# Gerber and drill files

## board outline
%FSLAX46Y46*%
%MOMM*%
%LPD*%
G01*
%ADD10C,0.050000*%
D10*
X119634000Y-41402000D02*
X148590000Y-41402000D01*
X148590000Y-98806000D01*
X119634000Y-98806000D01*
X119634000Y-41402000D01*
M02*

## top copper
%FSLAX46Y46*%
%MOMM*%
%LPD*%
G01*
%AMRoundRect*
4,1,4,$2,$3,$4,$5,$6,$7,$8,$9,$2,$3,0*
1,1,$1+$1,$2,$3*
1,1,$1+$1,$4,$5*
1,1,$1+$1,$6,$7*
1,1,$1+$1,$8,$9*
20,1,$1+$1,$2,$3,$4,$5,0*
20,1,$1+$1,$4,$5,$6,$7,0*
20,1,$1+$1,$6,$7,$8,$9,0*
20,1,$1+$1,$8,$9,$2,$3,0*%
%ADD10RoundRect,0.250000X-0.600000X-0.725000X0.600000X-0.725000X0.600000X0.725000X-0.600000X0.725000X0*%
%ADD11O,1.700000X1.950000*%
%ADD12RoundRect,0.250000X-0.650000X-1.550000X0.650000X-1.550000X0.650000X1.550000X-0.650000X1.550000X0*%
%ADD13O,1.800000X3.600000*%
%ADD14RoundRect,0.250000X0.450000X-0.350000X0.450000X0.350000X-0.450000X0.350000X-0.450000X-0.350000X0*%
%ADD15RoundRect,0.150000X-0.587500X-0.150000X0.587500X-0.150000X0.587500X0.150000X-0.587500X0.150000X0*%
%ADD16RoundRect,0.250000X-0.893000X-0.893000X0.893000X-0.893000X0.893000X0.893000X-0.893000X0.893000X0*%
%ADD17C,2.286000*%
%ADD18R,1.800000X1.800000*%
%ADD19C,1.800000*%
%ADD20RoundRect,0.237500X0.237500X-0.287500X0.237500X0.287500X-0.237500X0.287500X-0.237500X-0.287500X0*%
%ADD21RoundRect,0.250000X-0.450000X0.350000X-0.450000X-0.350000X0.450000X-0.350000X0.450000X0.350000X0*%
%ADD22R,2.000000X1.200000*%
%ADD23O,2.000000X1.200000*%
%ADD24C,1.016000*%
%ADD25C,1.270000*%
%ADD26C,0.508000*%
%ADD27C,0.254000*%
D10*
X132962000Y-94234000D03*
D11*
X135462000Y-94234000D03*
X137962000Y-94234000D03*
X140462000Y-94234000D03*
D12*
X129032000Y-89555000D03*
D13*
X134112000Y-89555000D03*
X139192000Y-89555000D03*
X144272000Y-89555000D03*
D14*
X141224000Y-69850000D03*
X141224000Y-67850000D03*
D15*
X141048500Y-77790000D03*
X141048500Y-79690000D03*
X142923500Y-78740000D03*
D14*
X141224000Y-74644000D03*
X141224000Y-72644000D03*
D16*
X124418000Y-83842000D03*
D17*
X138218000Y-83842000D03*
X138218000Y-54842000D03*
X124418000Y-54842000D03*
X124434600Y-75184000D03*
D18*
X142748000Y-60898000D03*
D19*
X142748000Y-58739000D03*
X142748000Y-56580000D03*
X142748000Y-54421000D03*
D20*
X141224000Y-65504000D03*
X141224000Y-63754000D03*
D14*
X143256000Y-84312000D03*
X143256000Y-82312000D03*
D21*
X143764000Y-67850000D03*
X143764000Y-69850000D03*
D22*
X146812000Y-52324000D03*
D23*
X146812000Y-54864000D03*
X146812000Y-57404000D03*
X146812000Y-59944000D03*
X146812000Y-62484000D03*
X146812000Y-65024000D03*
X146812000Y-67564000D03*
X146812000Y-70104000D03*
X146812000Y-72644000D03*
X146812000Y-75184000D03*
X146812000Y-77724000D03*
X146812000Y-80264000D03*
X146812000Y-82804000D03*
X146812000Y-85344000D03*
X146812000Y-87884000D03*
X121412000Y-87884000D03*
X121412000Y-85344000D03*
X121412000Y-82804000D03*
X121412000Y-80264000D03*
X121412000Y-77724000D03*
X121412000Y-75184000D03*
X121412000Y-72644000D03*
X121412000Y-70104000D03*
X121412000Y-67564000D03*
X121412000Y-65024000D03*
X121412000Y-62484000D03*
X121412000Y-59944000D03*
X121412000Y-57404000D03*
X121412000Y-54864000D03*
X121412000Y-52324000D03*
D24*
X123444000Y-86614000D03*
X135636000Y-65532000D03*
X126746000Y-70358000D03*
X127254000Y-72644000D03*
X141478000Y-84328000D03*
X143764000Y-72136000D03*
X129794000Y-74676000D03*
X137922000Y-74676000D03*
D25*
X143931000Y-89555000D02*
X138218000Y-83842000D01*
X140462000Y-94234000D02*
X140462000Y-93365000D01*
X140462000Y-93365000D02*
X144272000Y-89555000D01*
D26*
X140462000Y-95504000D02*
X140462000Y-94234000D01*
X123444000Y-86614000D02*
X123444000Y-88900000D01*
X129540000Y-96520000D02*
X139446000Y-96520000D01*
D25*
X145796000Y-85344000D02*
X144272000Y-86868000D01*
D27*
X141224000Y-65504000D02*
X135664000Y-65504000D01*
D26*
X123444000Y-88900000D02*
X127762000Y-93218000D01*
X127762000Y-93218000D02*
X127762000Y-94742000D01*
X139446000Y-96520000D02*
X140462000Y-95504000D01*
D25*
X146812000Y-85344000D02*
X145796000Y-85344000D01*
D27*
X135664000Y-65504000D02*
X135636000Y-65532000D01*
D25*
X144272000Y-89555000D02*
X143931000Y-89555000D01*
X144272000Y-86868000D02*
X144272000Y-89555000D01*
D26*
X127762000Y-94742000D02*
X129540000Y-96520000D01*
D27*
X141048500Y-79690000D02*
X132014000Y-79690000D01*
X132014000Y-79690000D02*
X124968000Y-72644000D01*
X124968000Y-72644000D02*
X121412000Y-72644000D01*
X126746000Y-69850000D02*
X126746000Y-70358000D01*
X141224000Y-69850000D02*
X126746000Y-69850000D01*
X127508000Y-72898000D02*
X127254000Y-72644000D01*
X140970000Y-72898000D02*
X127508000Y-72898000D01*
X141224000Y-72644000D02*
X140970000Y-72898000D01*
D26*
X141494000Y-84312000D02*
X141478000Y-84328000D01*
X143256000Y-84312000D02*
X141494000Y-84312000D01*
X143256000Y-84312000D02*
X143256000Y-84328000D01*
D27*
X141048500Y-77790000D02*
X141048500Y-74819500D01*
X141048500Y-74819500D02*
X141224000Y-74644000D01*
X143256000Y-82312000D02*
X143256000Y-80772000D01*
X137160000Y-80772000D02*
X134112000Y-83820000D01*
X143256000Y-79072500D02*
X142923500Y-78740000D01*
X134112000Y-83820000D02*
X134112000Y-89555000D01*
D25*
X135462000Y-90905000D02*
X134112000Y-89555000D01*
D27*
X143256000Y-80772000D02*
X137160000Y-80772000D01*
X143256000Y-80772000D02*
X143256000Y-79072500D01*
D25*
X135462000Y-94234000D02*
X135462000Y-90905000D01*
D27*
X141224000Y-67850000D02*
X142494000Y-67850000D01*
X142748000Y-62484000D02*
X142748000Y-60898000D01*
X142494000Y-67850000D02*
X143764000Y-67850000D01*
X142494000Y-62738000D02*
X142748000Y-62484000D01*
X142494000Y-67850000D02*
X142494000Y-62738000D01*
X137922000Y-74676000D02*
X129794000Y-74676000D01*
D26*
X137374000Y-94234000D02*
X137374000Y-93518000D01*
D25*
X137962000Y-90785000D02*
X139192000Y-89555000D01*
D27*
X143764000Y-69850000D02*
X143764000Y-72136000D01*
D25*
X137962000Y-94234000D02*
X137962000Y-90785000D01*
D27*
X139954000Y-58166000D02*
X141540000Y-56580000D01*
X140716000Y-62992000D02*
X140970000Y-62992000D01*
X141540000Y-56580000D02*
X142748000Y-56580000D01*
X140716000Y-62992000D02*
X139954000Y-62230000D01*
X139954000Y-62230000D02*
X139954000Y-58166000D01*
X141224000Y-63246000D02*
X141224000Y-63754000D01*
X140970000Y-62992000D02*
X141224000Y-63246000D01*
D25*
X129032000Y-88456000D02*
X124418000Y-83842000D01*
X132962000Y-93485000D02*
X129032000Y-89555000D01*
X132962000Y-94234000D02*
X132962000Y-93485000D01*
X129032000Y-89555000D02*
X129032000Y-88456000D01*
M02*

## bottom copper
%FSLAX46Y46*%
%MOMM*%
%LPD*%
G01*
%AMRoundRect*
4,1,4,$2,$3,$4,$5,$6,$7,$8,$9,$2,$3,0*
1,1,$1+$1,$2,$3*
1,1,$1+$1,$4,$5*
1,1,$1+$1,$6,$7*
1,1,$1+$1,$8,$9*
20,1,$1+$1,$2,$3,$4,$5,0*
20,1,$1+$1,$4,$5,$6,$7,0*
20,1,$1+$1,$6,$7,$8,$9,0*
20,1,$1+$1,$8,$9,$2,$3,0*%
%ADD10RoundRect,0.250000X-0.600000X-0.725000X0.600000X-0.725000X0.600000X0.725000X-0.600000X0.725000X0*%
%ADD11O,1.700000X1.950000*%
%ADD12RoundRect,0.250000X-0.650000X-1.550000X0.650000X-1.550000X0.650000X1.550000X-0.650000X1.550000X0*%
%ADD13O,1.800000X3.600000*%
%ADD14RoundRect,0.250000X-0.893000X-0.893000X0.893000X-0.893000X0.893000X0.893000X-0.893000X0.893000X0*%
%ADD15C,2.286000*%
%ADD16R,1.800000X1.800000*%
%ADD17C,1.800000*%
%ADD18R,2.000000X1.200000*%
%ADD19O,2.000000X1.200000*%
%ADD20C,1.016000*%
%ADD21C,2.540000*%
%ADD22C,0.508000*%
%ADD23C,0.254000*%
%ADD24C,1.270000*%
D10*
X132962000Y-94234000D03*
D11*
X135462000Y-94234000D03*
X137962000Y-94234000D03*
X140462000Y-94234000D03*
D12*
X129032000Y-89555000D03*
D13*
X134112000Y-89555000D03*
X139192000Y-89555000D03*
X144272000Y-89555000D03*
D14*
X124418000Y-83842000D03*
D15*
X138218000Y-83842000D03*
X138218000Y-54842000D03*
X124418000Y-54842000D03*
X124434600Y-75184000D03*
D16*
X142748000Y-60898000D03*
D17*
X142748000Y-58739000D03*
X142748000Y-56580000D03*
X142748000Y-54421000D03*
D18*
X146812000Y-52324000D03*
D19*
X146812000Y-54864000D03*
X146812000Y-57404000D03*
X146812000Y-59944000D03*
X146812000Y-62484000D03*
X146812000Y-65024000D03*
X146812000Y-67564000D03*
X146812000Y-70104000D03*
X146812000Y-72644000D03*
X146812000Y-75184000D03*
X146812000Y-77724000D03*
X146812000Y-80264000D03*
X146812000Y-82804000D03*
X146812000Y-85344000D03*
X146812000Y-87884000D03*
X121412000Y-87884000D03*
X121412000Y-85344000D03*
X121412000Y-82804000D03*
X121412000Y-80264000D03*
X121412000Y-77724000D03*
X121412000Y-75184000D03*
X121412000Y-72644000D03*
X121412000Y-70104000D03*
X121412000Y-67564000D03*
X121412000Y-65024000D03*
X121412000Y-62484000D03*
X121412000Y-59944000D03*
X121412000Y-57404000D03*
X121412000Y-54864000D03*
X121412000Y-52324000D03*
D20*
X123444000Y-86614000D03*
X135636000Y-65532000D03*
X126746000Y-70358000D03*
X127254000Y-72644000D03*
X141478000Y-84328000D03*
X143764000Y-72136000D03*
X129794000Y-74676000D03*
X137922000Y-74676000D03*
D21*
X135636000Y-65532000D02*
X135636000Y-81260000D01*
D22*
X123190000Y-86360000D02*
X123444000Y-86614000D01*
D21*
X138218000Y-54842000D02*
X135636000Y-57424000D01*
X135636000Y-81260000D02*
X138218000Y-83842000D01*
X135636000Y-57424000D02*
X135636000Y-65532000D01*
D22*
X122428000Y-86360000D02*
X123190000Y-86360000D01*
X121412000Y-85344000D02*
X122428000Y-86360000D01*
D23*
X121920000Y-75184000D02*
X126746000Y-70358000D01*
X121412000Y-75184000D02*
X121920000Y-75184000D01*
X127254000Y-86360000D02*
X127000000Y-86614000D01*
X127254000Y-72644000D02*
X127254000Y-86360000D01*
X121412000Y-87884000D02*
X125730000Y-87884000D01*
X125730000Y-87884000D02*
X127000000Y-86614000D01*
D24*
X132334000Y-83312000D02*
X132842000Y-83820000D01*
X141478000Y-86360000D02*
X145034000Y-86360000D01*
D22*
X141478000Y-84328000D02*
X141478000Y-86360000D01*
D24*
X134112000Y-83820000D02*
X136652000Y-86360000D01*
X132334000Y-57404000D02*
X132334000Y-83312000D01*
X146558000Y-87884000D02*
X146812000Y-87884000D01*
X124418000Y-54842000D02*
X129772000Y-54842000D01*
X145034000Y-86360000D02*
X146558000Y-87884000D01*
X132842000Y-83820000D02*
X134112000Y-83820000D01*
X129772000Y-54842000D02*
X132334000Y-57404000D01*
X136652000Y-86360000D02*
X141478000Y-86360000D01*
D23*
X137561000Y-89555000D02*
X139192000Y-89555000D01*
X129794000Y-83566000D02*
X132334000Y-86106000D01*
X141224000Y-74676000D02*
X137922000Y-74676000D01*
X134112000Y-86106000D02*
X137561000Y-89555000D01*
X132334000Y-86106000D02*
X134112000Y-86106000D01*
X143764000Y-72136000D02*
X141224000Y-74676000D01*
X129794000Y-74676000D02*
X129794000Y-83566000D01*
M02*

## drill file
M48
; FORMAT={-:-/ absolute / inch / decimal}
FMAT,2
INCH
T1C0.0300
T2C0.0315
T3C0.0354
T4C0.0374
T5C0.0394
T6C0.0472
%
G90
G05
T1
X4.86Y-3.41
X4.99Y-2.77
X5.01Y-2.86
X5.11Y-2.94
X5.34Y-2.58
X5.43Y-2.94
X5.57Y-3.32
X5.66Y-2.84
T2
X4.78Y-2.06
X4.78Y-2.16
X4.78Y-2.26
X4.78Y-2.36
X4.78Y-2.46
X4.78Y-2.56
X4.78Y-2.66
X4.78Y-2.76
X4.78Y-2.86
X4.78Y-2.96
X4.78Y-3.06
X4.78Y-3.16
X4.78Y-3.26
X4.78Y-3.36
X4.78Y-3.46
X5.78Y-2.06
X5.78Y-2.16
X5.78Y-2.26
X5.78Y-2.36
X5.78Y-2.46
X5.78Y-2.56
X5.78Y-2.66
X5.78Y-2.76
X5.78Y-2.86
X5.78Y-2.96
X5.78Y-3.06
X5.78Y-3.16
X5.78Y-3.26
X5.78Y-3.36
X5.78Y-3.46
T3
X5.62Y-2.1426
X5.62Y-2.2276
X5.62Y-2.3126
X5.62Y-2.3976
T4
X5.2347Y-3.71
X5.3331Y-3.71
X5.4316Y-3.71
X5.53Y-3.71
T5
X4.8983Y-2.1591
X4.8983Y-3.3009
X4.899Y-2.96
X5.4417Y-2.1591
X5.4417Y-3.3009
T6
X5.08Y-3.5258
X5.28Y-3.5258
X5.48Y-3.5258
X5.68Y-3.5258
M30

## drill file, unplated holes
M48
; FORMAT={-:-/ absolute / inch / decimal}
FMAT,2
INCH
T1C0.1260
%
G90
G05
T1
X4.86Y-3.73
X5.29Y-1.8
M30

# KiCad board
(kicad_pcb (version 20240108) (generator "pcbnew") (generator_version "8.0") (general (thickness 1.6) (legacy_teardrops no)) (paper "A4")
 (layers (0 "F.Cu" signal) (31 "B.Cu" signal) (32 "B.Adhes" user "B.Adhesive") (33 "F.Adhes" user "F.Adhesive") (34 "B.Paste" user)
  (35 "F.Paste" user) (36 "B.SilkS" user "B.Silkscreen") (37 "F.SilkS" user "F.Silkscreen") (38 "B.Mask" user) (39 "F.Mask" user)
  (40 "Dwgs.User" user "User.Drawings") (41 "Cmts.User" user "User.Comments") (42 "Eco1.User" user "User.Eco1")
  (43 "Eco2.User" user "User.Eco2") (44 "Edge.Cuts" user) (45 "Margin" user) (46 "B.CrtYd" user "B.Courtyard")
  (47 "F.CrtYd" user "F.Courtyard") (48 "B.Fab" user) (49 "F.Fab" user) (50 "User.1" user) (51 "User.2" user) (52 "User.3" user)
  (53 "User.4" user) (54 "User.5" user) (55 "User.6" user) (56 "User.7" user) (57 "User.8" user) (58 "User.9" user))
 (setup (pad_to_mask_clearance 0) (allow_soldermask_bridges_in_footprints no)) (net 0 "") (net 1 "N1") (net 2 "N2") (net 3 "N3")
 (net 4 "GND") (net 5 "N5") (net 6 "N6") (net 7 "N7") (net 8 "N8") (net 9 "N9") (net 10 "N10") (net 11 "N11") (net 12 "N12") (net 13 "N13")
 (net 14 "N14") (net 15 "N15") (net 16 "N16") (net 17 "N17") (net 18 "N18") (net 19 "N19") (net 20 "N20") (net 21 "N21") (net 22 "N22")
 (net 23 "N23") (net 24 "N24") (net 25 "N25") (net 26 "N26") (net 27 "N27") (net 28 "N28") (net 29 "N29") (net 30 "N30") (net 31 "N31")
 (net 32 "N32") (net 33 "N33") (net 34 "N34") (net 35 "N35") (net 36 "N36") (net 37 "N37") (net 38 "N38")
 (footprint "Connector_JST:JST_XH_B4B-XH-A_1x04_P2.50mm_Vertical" (layer "F.Cu") (at 132.962 94.234)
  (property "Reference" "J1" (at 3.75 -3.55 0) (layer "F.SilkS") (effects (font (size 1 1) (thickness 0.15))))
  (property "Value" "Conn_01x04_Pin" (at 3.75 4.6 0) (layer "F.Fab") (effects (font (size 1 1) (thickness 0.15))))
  (pad "1" thru_hole roundrect (at 0 0) (size 1.7 1.95) (drill 0.95) (layers "*.Cu" "*.Mask") (remove_unused_layers no)
   (roundrect_rratio 0.147059) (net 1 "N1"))
  (pad "2" thru_hole oval (at 2.5 0) (size 1.7 1.95) (drill 0.95) (layers "*.Cu" "*.Mask") (remove_unused_layers no) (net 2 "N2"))
  (pad "3" thru_hole oval (at 5 0) (size 1.7 1.95) (drill 0.95) (layers "*.Cu" "*.Mask") (remove_unused_layers no) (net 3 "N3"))
  (pad "4" thru_hole oval (at 7.5 0) (size 1.7 1.95) (drill 0.95) (layers "*.Cu" "*.Mask") (remove_unused_layers no) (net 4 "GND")))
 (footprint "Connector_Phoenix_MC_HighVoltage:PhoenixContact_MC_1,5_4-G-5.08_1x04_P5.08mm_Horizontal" (layer "F.Cu") (at 129.032 89.555)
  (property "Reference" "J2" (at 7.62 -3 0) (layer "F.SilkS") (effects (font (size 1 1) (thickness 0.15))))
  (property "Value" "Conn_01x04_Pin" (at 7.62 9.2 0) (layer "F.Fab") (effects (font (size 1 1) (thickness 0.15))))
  (pad "1" thru_hole roundrect (at 0 0) (size 1.8 3.6) (drill 1.2) (layers "*.Cu" "*.Mask") (remove_unused_layers no)
   (roundrect_rratio 0.138889) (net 1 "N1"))
  (pad "2" thru_hole oval (at 5.08 0) (size 1.8 3.6) (drill 1.2) (layers "*.Cu" "*.Mask") (remove_unused_layers no) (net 2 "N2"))
  (pad "3" thru_hole oval (at 10.16 0) (size 1.8 3.6) (drill 1.2) (layers "*.Cu" "*.Mask") (remove_unused_layers no) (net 3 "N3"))
  (pad "4" thru_hole oval (at 15.24 0) (size 1.8 3.6) (drill 1.2) (layers "*.Cu" "*.Mask") (remove_unused_layers no) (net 4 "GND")))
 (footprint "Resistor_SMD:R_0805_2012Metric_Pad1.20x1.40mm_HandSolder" (layer "F.Cu") (at 141.224 68.85 90)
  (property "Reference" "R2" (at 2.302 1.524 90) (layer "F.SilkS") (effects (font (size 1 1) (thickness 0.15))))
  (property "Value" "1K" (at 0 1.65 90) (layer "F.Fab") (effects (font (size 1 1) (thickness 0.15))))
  (pad "1" smd roundrect (at -1 0 90) (size 1.2 1.4) (layers "F.Cu" "F.Paste" "F.Mask") (roundrect_rratio 0.208333) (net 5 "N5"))
  (pad "2" smd roundrect (at 1 0 90) (size 1.2 1.4) (layers "F.Cu" "F.Paste" "F.Mask") (roundrect_rratio 0.208333) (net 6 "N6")))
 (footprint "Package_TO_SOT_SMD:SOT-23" (layer "F.Cu") (at 141.986 78.74)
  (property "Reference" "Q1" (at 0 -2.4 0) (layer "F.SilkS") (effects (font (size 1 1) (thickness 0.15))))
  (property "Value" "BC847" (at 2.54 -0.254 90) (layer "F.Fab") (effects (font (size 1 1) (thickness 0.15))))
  (pad "1" smd roundrect (at -0.9375 -0.95) (size 1.475 0.6) (layers "F.Cu" "F.Paste" "F.Mask") (roundrect_rratio 0.25) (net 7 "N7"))
  (pad "2" smd roundrect (at -0.9375 0.95) (size 1.475 0.6) (layers "F.Cu" "F.Paste" "F.Mask") (roundrect_rratio 0.25) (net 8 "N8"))
  (pad "3" smd roundrect (at 0.9375 0) (size 1.475 0.6) (layers "F.Cu" "F.Paste" "F.Mask") (roundrect_rratio 0.25) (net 2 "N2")))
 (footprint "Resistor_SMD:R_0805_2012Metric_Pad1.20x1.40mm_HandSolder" (layer "F.Cu") (at 141.224 73.644 90)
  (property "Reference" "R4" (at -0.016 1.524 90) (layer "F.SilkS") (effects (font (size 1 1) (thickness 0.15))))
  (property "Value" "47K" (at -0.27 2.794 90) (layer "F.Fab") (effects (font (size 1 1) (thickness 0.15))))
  (pad "1" smd roundrect (at -1 0 90) (size 1.2 1.4) (layers "F.Cu" "F.Paste" "F.Mask") (roundrect_rratio 0.208333) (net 7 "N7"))
  (pad "2" smd roundrect (at 1 0 90) (size 1.2 1.4) (layers "F.Cu" "F.Paste" "F.Mask") (roundrect_rratio 0.208333) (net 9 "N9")))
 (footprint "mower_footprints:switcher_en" (layer "F.Cu") (at 131.318 69.342)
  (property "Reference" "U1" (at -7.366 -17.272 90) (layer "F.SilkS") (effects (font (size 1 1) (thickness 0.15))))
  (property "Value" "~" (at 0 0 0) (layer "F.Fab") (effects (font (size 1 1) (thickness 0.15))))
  (pad "1" thru_hole roundrect (at -6.9 14.5) (size 2.286 2.286) (drill 1) (layers "*.Cu" "*.Mask") (remove_unused_layers no)
   (roundrect_rratio 0.1093613298) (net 1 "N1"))
  (pad "2" thru_hole circle (at 6.9 14.5) (size 2.286 2.286) (drill 1) (layers "*.Cu" "*.Mask") (remove_unused_layers no) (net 4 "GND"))
  (pad "3" thru_hole circle (at 6.9 -14.5) (size 2.286 2.286) (drill 1) (layers "*.Cu" "*.Mask") (remove_unused_layers no) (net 4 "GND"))
  (pad "4" thru_hole circle (at -6.9 -14.5) (size 2.286 2.286) (drill 1) (layers "*.Cu" "*.Mask") (remove_unused_layers no) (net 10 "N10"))
  (pad "5" thru_hole circle (at -6.8834 5.842) (size 2.286 2.286) (drill 1) (layers "*.Cu" "*.Mask") (remove_unused_layers no)
   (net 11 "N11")))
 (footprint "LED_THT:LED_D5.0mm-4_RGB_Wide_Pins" (layer "F.Cu") (at 142.748 60.898 90)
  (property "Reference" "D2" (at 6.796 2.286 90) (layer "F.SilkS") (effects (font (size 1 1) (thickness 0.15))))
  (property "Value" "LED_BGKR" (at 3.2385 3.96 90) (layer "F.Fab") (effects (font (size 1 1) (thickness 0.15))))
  (pad "1" thru_hole rect (at 0 0 90) (size 1.8 1.8) (drill 0.9) (layers "*.Cu" "*.Mask") (remove_unused_layers no) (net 6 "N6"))
  (pad "2" thru_hole circle (at 2.159 0 90) (size 1.8 1.8) (drill 0.9) (layers "*.Cu" "*.Mask") (remove_unused_layers no) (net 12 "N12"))
  (pad "3" thru_hole circle (at 4.318 0 90) (size 1.8 1.8) (drill 0.9) (layers "*.Cu" "*.Mask") (remove_unused_layers no) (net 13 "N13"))
  (pad "4" thru_hole circle (at 6.477 0 90) (size 1.8 1.8) (drill 0.9) (layers "*.Cu" "*.Mask") (remove_unused_layers no) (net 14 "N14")))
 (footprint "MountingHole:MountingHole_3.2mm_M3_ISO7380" (layer "F.Cu") (at 134.366 45.72)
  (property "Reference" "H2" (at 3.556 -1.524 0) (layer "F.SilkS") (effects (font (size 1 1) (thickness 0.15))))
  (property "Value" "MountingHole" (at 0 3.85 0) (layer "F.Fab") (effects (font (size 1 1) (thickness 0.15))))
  (pad "" np_thru_hole circle (at 0 0) (size 3.2 3.2) (drill 3.2) (layers "*.Cu" "*.Mask")))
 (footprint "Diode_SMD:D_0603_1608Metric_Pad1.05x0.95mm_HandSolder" (layer "F.Cu") (at 141.224 64.629 90)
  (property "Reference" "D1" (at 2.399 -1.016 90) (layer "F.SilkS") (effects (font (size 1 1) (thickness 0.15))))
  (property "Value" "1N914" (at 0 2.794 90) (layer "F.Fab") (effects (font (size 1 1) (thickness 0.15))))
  (pad "1" smd roundrect (at -0.875 0 90) (size 1.05 0.95) (layers "F.Cu" "F.Paste" "F.Mask") (roundrect_rratio 0.25) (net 4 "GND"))
  (pad "2" smd roundrect (at 0.875 0 90) (size 1.05 0.95) (layers "F.Cu" "F.Paste" "F.Mask") (roundrect_rratio 0.25) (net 13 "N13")))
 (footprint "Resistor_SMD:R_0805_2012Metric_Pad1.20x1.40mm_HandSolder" (layer "F.Cu") (at 143.256 83.312 90)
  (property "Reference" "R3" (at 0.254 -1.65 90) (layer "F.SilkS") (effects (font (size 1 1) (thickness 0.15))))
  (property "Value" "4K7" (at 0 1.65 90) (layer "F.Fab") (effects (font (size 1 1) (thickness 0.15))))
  (pad "1" smd roundrect (at -1 0 90) (size 1.2 1.4) (layers "F.Cu" "F.Paste" "F.Mask") (roundrect_rratio 0.208333) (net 10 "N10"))
  (pad "2" smd roundrect (at 1 0 90) (size 1.2 1.4) (layers "F.Cu" "F.Paste" "F.Mask") (roundrect_rratio 0.208333) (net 2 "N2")))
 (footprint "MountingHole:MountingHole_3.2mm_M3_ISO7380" (layer "F.Cu") (at 123.444 94.742)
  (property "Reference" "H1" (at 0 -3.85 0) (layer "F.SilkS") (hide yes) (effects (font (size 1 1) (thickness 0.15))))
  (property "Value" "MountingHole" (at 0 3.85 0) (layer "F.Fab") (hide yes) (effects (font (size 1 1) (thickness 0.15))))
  (pad "" np_thru_hole circle (at 0 0) (size 3.2 3.2) (drill 3.2) (layers "*.Cu" "*.Mask")))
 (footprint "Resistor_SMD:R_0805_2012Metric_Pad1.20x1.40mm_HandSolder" (layer "F.Cu") (at 143.764 68.85 -90)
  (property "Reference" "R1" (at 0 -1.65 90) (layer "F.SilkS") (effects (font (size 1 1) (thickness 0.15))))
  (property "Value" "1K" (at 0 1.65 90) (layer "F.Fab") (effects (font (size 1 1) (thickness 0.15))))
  (pad "1" smd roundrect (at -1 0 270) (size 1.2 1.4) (layers "F.Cu" "F.Paste" "F.Mask") (roundrect_rratio 0.208333) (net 6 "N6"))
  (pad "2" smd roundrect (at 1 0 270) (size 1.2 1.4) (layers "F.Cu" "F.Paste" "F.Mask") (roundrect_rratio 0.208333) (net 3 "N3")))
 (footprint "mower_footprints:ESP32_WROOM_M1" (layer "B.Cu") (at 134.112 70.104 -90)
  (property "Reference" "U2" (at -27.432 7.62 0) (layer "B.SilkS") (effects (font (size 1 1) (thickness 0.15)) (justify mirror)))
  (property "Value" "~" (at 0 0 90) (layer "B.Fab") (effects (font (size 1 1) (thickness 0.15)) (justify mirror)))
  (pad "1" thru_hole rect (at -17.78 -12.7 270) (size 1.2 2) (drill 0.8) (layers "*.Cu" "*.Mask") (remove_unused_layers no) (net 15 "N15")
   (thermal_bridge_angle 45))
  (pad "2" thru_hole oval (at -15.24 -12.7 270) (size 1.2 2) (drill 0.8) (layers "*.Cu" "*.Mask") (remove_unused_layers no) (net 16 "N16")
   (thermal_bridge_angle 45))
  (pad "3" thru_hole oval (at -12.7 -12.7 270) (size 1.2 2) (drill 0.8) (layers "*.Cu" "*.Mask") (remove_unused_layers no) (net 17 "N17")
   (thermal_bridge_angle 45))
  (pad "4" thru_hole oval (at -10.16 -12.7 270) (size 1.2 2) (drill 0.8) (layers "*.Cu" "*.Mask") (remove_unused_layers no) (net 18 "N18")
   (thermal_bridge_angle 45))
  (pad "5" thru_hole oval (at -7.62 -12.7 270) (size 1.2 2) (drill 0.8) (layers "*.Cu" "*.Mask") (remove_unused_layers no) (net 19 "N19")
   (thermal_bridge_angle 45))
  (pad "6" thru_hole oval (at -5.08 -12.7 270) (size 1.2 2) (drill 0.8) (layers "*.Cu" "*.Mask") (remove_unused_layers no) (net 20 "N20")
   (thermal_bridge_angle 45))
  (pad "7" thru_hole oval (at -2.54 -12.7 270) (size 1.2 2) (drill 0.8) (layers "*.Cu" "*.Mask") (remove_unused_layers no) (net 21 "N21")
   (thermal_bridge_angle 45))
  (pad "8" thru_hole oval (at 0 -12.7 270) (size 1.2 2) (drill 0.8) (layers "*.Cu" "*.Mask") (remove_unused_layers no) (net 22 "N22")
   (thermal_bridge_angle 45))
  (pad "9" thru_hole oval (at 2.54 -12.7 270) (size 1.2 2) (drill 0.8) (layers "*.Cu" "*.Mask") (remove_unused_layers no) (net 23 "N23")
   (thermal_bridge_angle 45))
  (pad "10" thru_hole oval (at 5.08 -12.7 270) (size 1.2 2) (drill 0.8) (layers "*.Cu" "*.Mask") (remove_unused_layers no) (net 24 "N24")
   (thermal_bridge_angle 45))
  (pad "11" thru_hole oval (at 7.62 -12.7 270) (size 1.2 2) (drill 0.8) (layers "*.Cu" "*.Mask") (remove_unused_layers no) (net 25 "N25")
   (thermal_bridge_angle 45))
  (pad "12" thru_hole oval (at 10.16 -12.7 270) (size 1.2 2) (drill 0.8) (layers "*.Cu" "*.Mask") (remove_unused_layers no) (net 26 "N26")
   (thermal_bridge_angle 45))
  (pad "13" thru_hole oval (at 12.7 -12.7 270) (size 1.2 2) (drill 0.8) (layers "*.Cu" "*.Mask") (remove_unused_layers no) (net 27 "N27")
   (thermal_bridge_angle 45))
  (pad "14" thru_hole oval (at 15.24 -12.7 270) (size 1.2 2) (drill 0.8) (layers "*.Cu" "*.Mask") (remove_unused_layers no) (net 4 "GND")
   (thermal_bridge_angle 45))
  (pad "15" thru_hole oval (at 17.78 -12.7 270) (size 1.2 2) (drill 0.8) (layers "*.Cu" "*.Mask") (remove_unused_layers no) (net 10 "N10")
   (thermal_bridge_angle 45))
  (pad "16" thru_hole oval (at 17.78 12.7 270) (size 1.2 2) (drill 0.8) (layers "*.Cu" "*.Mask") (remove_unused_layers no) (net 9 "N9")
   (thermal_bridge_angle 45))
  (pad "17" thru_hole oval (at 15.24 12.7 270) (size 1.2 2) (drill 0.8) (layers "*.Cu" "*.Mask") (remove_unused_layers no) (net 4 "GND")
   (thermal_bridge_angle 45))
  (pad "18" thru_hole oval (at 12.7 12.7 270) (size 1.2 2) (drill 0.8) (layers "*.Cu" "*.Mask") (remove_unused_layers no) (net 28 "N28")
   (thermal_bridge_angle 45))
  (pad "19" thru_hole oval (at 10.16 12.7 270) (size 1.2 2) (drill 0.8) (layers "*.Cu" "*.Mask") (remove_unused_layers no) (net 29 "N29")
   (thermal_bridge_angle 45))
  (pad "20" thru_hole oval (at 7.62 12.7 270) (size 1.2 2) (drill 0.8) (layers "*.Cu" "*.Mask") (remove_unused_layers no) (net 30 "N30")
   (thermal_bridge_angle 45))
  (pad "21" thru_hole oval (at 5.08 12.7 270) (size 1.2 2) (drill 0.8) (layers "*.Cu" "*.Mask") (remove_unused_layers no) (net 5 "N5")
   (thermal_bridge_angle 45))
  (pad "22" thru_hole oval (at 2.54 12.7 270) (size 1.2 2) (drill 0.8) (layers "*.Cu" "*.Mask") (remove_unused_layers no) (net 8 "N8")
   (thermal_bridge_angle 45))
  (pad "23" thru_hole oval (at 0 12.7 270) (size 1.2 2) (drill 0.8) (layers "*.Cu" "*.Mask") (remove_unused_layers no) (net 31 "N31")
   (thermal_bridge_angle 45))
  (pad "24" thru_hole oval (at -2.54 12.7 270) (size 1.2 2) (drill 0.8) (layers "*.Cu" "*.Mask") (remove_unused_layers no) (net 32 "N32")
   (thermal_bridge_angle 45))
  (pad "25" thru_hole oval (at -5.08 12.7 270) (size 1.2 2) (drill 0.8) (layers "*.Cu" "*.Mask") (remove_unused_layers no) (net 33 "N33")
   (thermal_bridge_angle 45))
  (pad "26" thru_hole oval (at -7.62 12.7 270) (size 1.2 2) (drill 0.8) (layers "*.Cu" "*.Mask") (remove_unused_layers no) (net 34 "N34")
   (thermal_bridge_angle 45))
  (pad "27" thru_hole oval (at -10.16 12.7 270) (size 1.2 2) (drill 0.8) (layers "*.Cu" "*.Mask") (remove_unused_layers no) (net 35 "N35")
   (thermal_bridge_angle 45))
  (pad "28" thru_hole oval (at -12.7 12.7 270) (size 1.2 2) (drill 0.8) (layers "*.Cu" "*.Mask") (remove_unused_layers no) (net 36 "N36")
   (thermal_bridge_angle 45))
  (pad "29" thru_hole oval (at -15.24 12.7 270) (size 1.2 2) (drill 0.8) (layers "*.Cu" "*.Mask") (remove_unused_layers no) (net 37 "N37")
   (thermal_bridge_angle 45))
  (pad "30" thru_hole oval (at -17.78 12.7 270) (size 1.2 2) (drill 0.8) (layers "*.Cu" "*.Mask") (remove_unused_layers no) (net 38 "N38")
   (thermal_bridge_angle 45)))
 (gr_rect (start 119.634 41.402) (end 148.59 98.806) (stroke (width 0.05) (type default)) (fill none) (layer "Edge.Cuts"))
 (segment (start 143.931 89.555) (end 138.218 83.842) (width 1.27) (layer "F.Cu") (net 4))
 (segment (start 140.462 94.234) (end 140.462 93.365) (width 1.27) (layer "F.Cu") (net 4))
 (segment (start 140.462 93.365) (end 144.272 89.555) (width 1.27) (layer "F.Cu") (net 4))
 (segment (start 140.462 95.504) (end 140.462 94.234) (width 0.508) (layer "F.Cu") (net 4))
 (segment (start 123.444 86.614) (end 123.444 88.9) (width 0.508) (layer "F.Cu") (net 4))
 (segment (start 129.54 96.52) (end 139.446 96.52) (width 0.508) (layer "F.Cu") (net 4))
 (segment (start 145.796 85.344) (end 144.272 86.868) (width 1.27) (layer "F.Cu") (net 4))
 (segment (start 141.224 65.504) (end 135.664 65.504) (width 0.254) (layer "F.Cu") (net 4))
 (segment (start 123.444 88.9) (end 127.762 93.218) (width 0.508) (layer "F.Cu") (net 4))
 (segment (start 127.762 93.218) (end 127.762 94.742) (width 0.508) (layer "F.Cu") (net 4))
 (segment (start 139.446 96.52) (end 140.462 95.504) (width 0.508) (layer "F.Cu") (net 4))
 (segment (start 146.812 85.344) (end 145.796 85.344) (width 1.27) (layer "F.Cu") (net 4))
 (segment (start 135.664 65.504) (end 135.636 65.532) (width 0.254) (layer "F.Cu") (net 4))
 (segment (start 144.272 89.555) (end 143.931 89.555) (width 1.27) (layer "F.Cu") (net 4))
 (segment (start 144.272 86.868) (end 144.272 89.555) (width 1.27) (layer "F.Cu") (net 4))
 (segment (start 127.762 94.742) (end 129.54 96.52) (width 0.508) (layer "F.Cu") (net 4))
 (via (at 123.444 86.614) (size 1.016) (drill 0.762) (layers "F.Cu" "B.Cu") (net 4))
 (via (at 135.636 65.532) (size 1.016) (drill 0.762) (layers "F.Cu" "B.Cu") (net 4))
 (segment (start 135.636 65.532) (end 135.636 81.26) (width 2.54) (layer "B.Cu") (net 4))
 (segment (start 123.19 86.36) (end 123.444 86.614) (width 0.508) (layer "B.Cu") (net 4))
 (segment (start 138.218 54.842) (end 135.636 57.424) (width 2.54) (layer "B.Cu") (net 4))
 (segment (start 135.636 81.26) (end 138.218 83.842) (width 2.54) (layer "B.Cu") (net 4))
 (segment (start 135.636 57.424) (end 135.636 65.532) (width 2.54) (layer "B.Cu") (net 4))
 (segment (start 122.428 86.36) (end 123.19 86.36) (width 0.508) (layer "B.Cu") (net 4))
 (segment (start 121.412 85.344) (end 122.428 86.36) (width 0.508) (layer "B.Cu") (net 4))
 (segment (start 141.0485 79.69) (end 132.014 79.69) (width 0.254) (layer "F.Cu") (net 8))
 (segment (start 132.014 79.69) (end 124.968 72.644) (width 0.254) (layer "F.Cu") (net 8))
 (segment (start 124.968 72.644) (end 121.412 72.644) (width 0.254) (layer "F.Cu") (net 8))
 (segment (start 126.746 69.85) (end 126.746 70.358) (width 0.254) (layer "F.Cu") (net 5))
 (segment (start 141.224 69.85) (end 126.746 69.85) (width 0.254) (layer "F.Cu") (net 5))
 (via (at 126.746 70.358) (size 1.016) (drill 0.762) (layers "F.Cu" "B.Cu") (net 5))
 (segment (start 121.92 75.184) (end 126.746 70.358) (width 0.254) (layer "B.Cu") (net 5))
 (segment (start 121.412 75.184) (end 121.92 75.184) (width 0.254) (layer "B.Cu") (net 5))
 (segment (start 127.508 72.898) (end 127.254 72.644) (width 0.254) (layer "F.Cu") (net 9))
 (segment (start 140.97 72.898) (end 127.508 72.898) (width 0.254) (layer "F.Cu") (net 9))
 (segment (start 141.224 72.644) (end 140.97 72.898) (width 0.254) (layer "F.Cu") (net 9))
 (via (at 127.254 72.644) (size 1.016) (drill 0.762) (layers "F.Cu" "B.Cu") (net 9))
 (segment (start 127.254 86.36) (end 127 86.614) (width 0.254) (layer "B.Cu") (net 9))
 (segment (start 127.254 72.644) (end 127.254 86.36) (width 0.254) (layer "B.Cu") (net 9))
 (segment (start 121.412 87.884) (end 125.73 87.884) (width 0.254) (layer "B.Cu") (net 9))
 (segment (start 125.73 87.884) (end 127 86.614) (width 0.254) (layer "B.Cu") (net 9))
 (segment (start 141.494 84.312) (end 141.478 84.328) (width 0.508) (layer "F.Cu") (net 10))
 (segment (start 143.256 84.312) (end 141.494 84.312) (width 0.508) (layer "F.Cu") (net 10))
 (segment (start 143.256 84.312) (end 143.256 84.328) (width 0.508) (layer "F.Cu") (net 10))
 (via (at 141.478 84.328) (size 1.016) (drill 0.762) (layers "F.Cu" "B.Cu") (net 10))
 (segment (start 132.334 83.312) (end 132.842 83.82) (width 1.27) (layer "B.Cu") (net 10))
 (segment (start 141.478 86.36) (end 145.034 86.36) (width 1.27) (layer "B.Cu") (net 10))
 (segment (start 141.478 84.328) (end 141.478 86.36) (width 0.508) (layer "B.Cu") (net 10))
 (segment (start 134.112 83.82) (end 136.652 86.36) (width 1.27) (layer "B.Cu") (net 10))
 (segment (start 132.334 57.404) (end 132.334 83.312) (width 1.27) (layer "B.Cu") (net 10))
 (segment (start 146.558 87.884) (end 146.812 87.884) (width 1.27) (layer "B.Cu") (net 10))
 (segment (start 124.418 54.842) (end 129.772 54.842) (width 1.27) (layer "B.Cu") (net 10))
 (segment (start 145.034 86.36) (end 146.558 87.884) (width 1.27) (layer "B.Cu") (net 10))
 (segment (start 132.842 83.82) (end 134.112 83.82) (width 1.27) (layer "B.Cu") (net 10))
 (segment (start 129.772 54.842) (end 132.334 57.404) (width 1.27) (layer "B.Cu") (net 10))
 (segment (start 136.652 86.36) (end 141.478 86.36) (width 1.27) (layer "B.Cu") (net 10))
 (segment (start 141.0485 77.79) (end 141.0485 74.8195) (width 0.254) (layer "F.Cu") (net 7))
 (segment (start 141.0485 74.8195) (end 141.224 74.644) (width 0.254) (layer "F.Cu") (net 7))
 (segment (start 143.256 82.312) (end 143.256 80.772) (width 0.254) (layer "F.Cu") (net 2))
 (segment (start 137.16 80.772) (end 134.112 83.82) (width 0.254) (layer "F.Cu") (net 2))
 (segment (start 143.256 79.0725) (end 142.9235 78.74) (width 0.254) (layer "F.Cu") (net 2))
 (segment (start 134.112 83.82) (end 134.112 89.555) (width 0.254) (layer "F.Cu") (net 2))
 (segment (start 135.462 90.905) (end 134.112 89.555) (width 1.27) (layer "F.Cu") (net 2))
 (segment (start 143.256 80.772) (end 137.16 80.772) (width 0.254) (layer "F.Cu") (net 2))
 (segment (start 143.256 80.772) (end 143.256 79.0725) (width 0.254) (layer "F.Cu") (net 2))
 (segment (start 135.462 94.234) (end 135.462 90.905) (width 1.27) (layer "F.Cu") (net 2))
 (segment (start 141.224 67.85) (end 142.494 67.85) (width 0.254) (layer "F.Cu") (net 6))
 (segment (start 142.748 62.484) (end 142.748 60.898) (width 0.254) (layer "F.Cu") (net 6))
 (segment (start 142.494 67.85) (end 143.764 67.85) (width 0.254) (layer "F.Cu") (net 6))
 (segment (start 142.494 62.738) (end 142.748 62.484) (width 0.254) (layer "F.Cu") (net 6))
 (segment (start 142.494 67.85) (end 142.494 62.738) (width 0.254) (layer "F.Cu") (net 6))
 (segment (start 137.922 74.676) (end 129.794 74.676) (width 0.254) (layer "F.Cu") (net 3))
 (segment (start 137.374 94.234) (end 137.374 93.518) (width 0.508) (layer "F.Cu") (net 3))
 (segment (start 137.962 90.785) (end 139.192 89.555) (width 1.27) (layer "F.Cu") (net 3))
 (segment (start 143.764 69.85) (end 143.764 72.136) (width 0.254) (layer "F.Cu") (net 3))
 (segment (start 137.962 94.234) (end 137.962 90.785) (width 1.27) (layer "F.Cu") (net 3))
 (via (at 143.764 72.136) (size 1.016) (drill 0.762) (layers "F.Cu" "B.Cu") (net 3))
 (via (at 129.794 74.676) (size 1.016) (drill 0.762) (layers "F.Cu" "B.Cu") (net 3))
 (via (at 137.922 74.676) (size 1.016) (drill 0.762) (layers "F.Cu" "B.Cu") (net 3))
 (segment (start 137.561 89.555) (end 139.192 89.555) (width 0.254) (layer "B.Cu") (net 3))
 (segment (start 129.794 83.566) (end 132.334 86.106) (width 0.254) (layer "B.Cu") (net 3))
 (segment (start 141.224 74.676) (end 137.922 74.676) (width 0.254) (layer "B.Cu") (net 3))
 (segment (start 134.112 86.106) (end 137.561 89.555) (width 0.254) (layer "B.Cu") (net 3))
 (segment (start 132.334 86.106) (end 134.112 86.106) (width 0.254) (layer "B.Cu") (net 3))
 (segment (start 143.764 72.136) (end 141.224 74.676) (width 0.254) (layer "B.Cu") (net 3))
 (segment (start 129.794 74.676) (end 129.794 83.566) (width 0.254) (layer "B.Cu") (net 3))
 (segment (start 139.954 58.166) (end 141.54 56.58) (width 0.254) (layer "F.Cu") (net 13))
 (segment (start 140.716 62.992) (end 140.97 62.992) (width 0.254) (layer "F.Cu") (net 13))
 (segment (start 141.54 56.58) (end 142.748 56.58) (width 0.254) (layer "F.Cu") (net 13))
 (segment (start 140.716 62.992) (end 139.954 62.23) (width 0.254) (layer "F.Cu") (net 13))
 (segment (start 139.954 62.23) (end 139.954 58.166) (width 0.254) (layer "F.Cu") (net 13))
 (segment (start 141.224 63.246) (end 141.224 63.754) (width 0.254) (layer "F.Cu") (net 13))
 (segment (start 140.97 62.992) (end 141.224 63.246) (width 0.254) (layer "F.Cu") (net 13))
 (segment (start 129.032 88.456) (end 124.418 83.842) (width 1.27) (layer "F.Cu") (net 1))
 (segment (start 132.962 93.485) (end 129.032 89.555) (width 1.27) (layer "F.Cu") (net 1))
 (segment (start 132.962 94.234) (end 132.962 93.485) (width 1.27) (layer "F.Cu") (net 1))
 (segment (start 129.032 89.555) (end 129.032 88.456) (width 1.27) (layer "F.Cu") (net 1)))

